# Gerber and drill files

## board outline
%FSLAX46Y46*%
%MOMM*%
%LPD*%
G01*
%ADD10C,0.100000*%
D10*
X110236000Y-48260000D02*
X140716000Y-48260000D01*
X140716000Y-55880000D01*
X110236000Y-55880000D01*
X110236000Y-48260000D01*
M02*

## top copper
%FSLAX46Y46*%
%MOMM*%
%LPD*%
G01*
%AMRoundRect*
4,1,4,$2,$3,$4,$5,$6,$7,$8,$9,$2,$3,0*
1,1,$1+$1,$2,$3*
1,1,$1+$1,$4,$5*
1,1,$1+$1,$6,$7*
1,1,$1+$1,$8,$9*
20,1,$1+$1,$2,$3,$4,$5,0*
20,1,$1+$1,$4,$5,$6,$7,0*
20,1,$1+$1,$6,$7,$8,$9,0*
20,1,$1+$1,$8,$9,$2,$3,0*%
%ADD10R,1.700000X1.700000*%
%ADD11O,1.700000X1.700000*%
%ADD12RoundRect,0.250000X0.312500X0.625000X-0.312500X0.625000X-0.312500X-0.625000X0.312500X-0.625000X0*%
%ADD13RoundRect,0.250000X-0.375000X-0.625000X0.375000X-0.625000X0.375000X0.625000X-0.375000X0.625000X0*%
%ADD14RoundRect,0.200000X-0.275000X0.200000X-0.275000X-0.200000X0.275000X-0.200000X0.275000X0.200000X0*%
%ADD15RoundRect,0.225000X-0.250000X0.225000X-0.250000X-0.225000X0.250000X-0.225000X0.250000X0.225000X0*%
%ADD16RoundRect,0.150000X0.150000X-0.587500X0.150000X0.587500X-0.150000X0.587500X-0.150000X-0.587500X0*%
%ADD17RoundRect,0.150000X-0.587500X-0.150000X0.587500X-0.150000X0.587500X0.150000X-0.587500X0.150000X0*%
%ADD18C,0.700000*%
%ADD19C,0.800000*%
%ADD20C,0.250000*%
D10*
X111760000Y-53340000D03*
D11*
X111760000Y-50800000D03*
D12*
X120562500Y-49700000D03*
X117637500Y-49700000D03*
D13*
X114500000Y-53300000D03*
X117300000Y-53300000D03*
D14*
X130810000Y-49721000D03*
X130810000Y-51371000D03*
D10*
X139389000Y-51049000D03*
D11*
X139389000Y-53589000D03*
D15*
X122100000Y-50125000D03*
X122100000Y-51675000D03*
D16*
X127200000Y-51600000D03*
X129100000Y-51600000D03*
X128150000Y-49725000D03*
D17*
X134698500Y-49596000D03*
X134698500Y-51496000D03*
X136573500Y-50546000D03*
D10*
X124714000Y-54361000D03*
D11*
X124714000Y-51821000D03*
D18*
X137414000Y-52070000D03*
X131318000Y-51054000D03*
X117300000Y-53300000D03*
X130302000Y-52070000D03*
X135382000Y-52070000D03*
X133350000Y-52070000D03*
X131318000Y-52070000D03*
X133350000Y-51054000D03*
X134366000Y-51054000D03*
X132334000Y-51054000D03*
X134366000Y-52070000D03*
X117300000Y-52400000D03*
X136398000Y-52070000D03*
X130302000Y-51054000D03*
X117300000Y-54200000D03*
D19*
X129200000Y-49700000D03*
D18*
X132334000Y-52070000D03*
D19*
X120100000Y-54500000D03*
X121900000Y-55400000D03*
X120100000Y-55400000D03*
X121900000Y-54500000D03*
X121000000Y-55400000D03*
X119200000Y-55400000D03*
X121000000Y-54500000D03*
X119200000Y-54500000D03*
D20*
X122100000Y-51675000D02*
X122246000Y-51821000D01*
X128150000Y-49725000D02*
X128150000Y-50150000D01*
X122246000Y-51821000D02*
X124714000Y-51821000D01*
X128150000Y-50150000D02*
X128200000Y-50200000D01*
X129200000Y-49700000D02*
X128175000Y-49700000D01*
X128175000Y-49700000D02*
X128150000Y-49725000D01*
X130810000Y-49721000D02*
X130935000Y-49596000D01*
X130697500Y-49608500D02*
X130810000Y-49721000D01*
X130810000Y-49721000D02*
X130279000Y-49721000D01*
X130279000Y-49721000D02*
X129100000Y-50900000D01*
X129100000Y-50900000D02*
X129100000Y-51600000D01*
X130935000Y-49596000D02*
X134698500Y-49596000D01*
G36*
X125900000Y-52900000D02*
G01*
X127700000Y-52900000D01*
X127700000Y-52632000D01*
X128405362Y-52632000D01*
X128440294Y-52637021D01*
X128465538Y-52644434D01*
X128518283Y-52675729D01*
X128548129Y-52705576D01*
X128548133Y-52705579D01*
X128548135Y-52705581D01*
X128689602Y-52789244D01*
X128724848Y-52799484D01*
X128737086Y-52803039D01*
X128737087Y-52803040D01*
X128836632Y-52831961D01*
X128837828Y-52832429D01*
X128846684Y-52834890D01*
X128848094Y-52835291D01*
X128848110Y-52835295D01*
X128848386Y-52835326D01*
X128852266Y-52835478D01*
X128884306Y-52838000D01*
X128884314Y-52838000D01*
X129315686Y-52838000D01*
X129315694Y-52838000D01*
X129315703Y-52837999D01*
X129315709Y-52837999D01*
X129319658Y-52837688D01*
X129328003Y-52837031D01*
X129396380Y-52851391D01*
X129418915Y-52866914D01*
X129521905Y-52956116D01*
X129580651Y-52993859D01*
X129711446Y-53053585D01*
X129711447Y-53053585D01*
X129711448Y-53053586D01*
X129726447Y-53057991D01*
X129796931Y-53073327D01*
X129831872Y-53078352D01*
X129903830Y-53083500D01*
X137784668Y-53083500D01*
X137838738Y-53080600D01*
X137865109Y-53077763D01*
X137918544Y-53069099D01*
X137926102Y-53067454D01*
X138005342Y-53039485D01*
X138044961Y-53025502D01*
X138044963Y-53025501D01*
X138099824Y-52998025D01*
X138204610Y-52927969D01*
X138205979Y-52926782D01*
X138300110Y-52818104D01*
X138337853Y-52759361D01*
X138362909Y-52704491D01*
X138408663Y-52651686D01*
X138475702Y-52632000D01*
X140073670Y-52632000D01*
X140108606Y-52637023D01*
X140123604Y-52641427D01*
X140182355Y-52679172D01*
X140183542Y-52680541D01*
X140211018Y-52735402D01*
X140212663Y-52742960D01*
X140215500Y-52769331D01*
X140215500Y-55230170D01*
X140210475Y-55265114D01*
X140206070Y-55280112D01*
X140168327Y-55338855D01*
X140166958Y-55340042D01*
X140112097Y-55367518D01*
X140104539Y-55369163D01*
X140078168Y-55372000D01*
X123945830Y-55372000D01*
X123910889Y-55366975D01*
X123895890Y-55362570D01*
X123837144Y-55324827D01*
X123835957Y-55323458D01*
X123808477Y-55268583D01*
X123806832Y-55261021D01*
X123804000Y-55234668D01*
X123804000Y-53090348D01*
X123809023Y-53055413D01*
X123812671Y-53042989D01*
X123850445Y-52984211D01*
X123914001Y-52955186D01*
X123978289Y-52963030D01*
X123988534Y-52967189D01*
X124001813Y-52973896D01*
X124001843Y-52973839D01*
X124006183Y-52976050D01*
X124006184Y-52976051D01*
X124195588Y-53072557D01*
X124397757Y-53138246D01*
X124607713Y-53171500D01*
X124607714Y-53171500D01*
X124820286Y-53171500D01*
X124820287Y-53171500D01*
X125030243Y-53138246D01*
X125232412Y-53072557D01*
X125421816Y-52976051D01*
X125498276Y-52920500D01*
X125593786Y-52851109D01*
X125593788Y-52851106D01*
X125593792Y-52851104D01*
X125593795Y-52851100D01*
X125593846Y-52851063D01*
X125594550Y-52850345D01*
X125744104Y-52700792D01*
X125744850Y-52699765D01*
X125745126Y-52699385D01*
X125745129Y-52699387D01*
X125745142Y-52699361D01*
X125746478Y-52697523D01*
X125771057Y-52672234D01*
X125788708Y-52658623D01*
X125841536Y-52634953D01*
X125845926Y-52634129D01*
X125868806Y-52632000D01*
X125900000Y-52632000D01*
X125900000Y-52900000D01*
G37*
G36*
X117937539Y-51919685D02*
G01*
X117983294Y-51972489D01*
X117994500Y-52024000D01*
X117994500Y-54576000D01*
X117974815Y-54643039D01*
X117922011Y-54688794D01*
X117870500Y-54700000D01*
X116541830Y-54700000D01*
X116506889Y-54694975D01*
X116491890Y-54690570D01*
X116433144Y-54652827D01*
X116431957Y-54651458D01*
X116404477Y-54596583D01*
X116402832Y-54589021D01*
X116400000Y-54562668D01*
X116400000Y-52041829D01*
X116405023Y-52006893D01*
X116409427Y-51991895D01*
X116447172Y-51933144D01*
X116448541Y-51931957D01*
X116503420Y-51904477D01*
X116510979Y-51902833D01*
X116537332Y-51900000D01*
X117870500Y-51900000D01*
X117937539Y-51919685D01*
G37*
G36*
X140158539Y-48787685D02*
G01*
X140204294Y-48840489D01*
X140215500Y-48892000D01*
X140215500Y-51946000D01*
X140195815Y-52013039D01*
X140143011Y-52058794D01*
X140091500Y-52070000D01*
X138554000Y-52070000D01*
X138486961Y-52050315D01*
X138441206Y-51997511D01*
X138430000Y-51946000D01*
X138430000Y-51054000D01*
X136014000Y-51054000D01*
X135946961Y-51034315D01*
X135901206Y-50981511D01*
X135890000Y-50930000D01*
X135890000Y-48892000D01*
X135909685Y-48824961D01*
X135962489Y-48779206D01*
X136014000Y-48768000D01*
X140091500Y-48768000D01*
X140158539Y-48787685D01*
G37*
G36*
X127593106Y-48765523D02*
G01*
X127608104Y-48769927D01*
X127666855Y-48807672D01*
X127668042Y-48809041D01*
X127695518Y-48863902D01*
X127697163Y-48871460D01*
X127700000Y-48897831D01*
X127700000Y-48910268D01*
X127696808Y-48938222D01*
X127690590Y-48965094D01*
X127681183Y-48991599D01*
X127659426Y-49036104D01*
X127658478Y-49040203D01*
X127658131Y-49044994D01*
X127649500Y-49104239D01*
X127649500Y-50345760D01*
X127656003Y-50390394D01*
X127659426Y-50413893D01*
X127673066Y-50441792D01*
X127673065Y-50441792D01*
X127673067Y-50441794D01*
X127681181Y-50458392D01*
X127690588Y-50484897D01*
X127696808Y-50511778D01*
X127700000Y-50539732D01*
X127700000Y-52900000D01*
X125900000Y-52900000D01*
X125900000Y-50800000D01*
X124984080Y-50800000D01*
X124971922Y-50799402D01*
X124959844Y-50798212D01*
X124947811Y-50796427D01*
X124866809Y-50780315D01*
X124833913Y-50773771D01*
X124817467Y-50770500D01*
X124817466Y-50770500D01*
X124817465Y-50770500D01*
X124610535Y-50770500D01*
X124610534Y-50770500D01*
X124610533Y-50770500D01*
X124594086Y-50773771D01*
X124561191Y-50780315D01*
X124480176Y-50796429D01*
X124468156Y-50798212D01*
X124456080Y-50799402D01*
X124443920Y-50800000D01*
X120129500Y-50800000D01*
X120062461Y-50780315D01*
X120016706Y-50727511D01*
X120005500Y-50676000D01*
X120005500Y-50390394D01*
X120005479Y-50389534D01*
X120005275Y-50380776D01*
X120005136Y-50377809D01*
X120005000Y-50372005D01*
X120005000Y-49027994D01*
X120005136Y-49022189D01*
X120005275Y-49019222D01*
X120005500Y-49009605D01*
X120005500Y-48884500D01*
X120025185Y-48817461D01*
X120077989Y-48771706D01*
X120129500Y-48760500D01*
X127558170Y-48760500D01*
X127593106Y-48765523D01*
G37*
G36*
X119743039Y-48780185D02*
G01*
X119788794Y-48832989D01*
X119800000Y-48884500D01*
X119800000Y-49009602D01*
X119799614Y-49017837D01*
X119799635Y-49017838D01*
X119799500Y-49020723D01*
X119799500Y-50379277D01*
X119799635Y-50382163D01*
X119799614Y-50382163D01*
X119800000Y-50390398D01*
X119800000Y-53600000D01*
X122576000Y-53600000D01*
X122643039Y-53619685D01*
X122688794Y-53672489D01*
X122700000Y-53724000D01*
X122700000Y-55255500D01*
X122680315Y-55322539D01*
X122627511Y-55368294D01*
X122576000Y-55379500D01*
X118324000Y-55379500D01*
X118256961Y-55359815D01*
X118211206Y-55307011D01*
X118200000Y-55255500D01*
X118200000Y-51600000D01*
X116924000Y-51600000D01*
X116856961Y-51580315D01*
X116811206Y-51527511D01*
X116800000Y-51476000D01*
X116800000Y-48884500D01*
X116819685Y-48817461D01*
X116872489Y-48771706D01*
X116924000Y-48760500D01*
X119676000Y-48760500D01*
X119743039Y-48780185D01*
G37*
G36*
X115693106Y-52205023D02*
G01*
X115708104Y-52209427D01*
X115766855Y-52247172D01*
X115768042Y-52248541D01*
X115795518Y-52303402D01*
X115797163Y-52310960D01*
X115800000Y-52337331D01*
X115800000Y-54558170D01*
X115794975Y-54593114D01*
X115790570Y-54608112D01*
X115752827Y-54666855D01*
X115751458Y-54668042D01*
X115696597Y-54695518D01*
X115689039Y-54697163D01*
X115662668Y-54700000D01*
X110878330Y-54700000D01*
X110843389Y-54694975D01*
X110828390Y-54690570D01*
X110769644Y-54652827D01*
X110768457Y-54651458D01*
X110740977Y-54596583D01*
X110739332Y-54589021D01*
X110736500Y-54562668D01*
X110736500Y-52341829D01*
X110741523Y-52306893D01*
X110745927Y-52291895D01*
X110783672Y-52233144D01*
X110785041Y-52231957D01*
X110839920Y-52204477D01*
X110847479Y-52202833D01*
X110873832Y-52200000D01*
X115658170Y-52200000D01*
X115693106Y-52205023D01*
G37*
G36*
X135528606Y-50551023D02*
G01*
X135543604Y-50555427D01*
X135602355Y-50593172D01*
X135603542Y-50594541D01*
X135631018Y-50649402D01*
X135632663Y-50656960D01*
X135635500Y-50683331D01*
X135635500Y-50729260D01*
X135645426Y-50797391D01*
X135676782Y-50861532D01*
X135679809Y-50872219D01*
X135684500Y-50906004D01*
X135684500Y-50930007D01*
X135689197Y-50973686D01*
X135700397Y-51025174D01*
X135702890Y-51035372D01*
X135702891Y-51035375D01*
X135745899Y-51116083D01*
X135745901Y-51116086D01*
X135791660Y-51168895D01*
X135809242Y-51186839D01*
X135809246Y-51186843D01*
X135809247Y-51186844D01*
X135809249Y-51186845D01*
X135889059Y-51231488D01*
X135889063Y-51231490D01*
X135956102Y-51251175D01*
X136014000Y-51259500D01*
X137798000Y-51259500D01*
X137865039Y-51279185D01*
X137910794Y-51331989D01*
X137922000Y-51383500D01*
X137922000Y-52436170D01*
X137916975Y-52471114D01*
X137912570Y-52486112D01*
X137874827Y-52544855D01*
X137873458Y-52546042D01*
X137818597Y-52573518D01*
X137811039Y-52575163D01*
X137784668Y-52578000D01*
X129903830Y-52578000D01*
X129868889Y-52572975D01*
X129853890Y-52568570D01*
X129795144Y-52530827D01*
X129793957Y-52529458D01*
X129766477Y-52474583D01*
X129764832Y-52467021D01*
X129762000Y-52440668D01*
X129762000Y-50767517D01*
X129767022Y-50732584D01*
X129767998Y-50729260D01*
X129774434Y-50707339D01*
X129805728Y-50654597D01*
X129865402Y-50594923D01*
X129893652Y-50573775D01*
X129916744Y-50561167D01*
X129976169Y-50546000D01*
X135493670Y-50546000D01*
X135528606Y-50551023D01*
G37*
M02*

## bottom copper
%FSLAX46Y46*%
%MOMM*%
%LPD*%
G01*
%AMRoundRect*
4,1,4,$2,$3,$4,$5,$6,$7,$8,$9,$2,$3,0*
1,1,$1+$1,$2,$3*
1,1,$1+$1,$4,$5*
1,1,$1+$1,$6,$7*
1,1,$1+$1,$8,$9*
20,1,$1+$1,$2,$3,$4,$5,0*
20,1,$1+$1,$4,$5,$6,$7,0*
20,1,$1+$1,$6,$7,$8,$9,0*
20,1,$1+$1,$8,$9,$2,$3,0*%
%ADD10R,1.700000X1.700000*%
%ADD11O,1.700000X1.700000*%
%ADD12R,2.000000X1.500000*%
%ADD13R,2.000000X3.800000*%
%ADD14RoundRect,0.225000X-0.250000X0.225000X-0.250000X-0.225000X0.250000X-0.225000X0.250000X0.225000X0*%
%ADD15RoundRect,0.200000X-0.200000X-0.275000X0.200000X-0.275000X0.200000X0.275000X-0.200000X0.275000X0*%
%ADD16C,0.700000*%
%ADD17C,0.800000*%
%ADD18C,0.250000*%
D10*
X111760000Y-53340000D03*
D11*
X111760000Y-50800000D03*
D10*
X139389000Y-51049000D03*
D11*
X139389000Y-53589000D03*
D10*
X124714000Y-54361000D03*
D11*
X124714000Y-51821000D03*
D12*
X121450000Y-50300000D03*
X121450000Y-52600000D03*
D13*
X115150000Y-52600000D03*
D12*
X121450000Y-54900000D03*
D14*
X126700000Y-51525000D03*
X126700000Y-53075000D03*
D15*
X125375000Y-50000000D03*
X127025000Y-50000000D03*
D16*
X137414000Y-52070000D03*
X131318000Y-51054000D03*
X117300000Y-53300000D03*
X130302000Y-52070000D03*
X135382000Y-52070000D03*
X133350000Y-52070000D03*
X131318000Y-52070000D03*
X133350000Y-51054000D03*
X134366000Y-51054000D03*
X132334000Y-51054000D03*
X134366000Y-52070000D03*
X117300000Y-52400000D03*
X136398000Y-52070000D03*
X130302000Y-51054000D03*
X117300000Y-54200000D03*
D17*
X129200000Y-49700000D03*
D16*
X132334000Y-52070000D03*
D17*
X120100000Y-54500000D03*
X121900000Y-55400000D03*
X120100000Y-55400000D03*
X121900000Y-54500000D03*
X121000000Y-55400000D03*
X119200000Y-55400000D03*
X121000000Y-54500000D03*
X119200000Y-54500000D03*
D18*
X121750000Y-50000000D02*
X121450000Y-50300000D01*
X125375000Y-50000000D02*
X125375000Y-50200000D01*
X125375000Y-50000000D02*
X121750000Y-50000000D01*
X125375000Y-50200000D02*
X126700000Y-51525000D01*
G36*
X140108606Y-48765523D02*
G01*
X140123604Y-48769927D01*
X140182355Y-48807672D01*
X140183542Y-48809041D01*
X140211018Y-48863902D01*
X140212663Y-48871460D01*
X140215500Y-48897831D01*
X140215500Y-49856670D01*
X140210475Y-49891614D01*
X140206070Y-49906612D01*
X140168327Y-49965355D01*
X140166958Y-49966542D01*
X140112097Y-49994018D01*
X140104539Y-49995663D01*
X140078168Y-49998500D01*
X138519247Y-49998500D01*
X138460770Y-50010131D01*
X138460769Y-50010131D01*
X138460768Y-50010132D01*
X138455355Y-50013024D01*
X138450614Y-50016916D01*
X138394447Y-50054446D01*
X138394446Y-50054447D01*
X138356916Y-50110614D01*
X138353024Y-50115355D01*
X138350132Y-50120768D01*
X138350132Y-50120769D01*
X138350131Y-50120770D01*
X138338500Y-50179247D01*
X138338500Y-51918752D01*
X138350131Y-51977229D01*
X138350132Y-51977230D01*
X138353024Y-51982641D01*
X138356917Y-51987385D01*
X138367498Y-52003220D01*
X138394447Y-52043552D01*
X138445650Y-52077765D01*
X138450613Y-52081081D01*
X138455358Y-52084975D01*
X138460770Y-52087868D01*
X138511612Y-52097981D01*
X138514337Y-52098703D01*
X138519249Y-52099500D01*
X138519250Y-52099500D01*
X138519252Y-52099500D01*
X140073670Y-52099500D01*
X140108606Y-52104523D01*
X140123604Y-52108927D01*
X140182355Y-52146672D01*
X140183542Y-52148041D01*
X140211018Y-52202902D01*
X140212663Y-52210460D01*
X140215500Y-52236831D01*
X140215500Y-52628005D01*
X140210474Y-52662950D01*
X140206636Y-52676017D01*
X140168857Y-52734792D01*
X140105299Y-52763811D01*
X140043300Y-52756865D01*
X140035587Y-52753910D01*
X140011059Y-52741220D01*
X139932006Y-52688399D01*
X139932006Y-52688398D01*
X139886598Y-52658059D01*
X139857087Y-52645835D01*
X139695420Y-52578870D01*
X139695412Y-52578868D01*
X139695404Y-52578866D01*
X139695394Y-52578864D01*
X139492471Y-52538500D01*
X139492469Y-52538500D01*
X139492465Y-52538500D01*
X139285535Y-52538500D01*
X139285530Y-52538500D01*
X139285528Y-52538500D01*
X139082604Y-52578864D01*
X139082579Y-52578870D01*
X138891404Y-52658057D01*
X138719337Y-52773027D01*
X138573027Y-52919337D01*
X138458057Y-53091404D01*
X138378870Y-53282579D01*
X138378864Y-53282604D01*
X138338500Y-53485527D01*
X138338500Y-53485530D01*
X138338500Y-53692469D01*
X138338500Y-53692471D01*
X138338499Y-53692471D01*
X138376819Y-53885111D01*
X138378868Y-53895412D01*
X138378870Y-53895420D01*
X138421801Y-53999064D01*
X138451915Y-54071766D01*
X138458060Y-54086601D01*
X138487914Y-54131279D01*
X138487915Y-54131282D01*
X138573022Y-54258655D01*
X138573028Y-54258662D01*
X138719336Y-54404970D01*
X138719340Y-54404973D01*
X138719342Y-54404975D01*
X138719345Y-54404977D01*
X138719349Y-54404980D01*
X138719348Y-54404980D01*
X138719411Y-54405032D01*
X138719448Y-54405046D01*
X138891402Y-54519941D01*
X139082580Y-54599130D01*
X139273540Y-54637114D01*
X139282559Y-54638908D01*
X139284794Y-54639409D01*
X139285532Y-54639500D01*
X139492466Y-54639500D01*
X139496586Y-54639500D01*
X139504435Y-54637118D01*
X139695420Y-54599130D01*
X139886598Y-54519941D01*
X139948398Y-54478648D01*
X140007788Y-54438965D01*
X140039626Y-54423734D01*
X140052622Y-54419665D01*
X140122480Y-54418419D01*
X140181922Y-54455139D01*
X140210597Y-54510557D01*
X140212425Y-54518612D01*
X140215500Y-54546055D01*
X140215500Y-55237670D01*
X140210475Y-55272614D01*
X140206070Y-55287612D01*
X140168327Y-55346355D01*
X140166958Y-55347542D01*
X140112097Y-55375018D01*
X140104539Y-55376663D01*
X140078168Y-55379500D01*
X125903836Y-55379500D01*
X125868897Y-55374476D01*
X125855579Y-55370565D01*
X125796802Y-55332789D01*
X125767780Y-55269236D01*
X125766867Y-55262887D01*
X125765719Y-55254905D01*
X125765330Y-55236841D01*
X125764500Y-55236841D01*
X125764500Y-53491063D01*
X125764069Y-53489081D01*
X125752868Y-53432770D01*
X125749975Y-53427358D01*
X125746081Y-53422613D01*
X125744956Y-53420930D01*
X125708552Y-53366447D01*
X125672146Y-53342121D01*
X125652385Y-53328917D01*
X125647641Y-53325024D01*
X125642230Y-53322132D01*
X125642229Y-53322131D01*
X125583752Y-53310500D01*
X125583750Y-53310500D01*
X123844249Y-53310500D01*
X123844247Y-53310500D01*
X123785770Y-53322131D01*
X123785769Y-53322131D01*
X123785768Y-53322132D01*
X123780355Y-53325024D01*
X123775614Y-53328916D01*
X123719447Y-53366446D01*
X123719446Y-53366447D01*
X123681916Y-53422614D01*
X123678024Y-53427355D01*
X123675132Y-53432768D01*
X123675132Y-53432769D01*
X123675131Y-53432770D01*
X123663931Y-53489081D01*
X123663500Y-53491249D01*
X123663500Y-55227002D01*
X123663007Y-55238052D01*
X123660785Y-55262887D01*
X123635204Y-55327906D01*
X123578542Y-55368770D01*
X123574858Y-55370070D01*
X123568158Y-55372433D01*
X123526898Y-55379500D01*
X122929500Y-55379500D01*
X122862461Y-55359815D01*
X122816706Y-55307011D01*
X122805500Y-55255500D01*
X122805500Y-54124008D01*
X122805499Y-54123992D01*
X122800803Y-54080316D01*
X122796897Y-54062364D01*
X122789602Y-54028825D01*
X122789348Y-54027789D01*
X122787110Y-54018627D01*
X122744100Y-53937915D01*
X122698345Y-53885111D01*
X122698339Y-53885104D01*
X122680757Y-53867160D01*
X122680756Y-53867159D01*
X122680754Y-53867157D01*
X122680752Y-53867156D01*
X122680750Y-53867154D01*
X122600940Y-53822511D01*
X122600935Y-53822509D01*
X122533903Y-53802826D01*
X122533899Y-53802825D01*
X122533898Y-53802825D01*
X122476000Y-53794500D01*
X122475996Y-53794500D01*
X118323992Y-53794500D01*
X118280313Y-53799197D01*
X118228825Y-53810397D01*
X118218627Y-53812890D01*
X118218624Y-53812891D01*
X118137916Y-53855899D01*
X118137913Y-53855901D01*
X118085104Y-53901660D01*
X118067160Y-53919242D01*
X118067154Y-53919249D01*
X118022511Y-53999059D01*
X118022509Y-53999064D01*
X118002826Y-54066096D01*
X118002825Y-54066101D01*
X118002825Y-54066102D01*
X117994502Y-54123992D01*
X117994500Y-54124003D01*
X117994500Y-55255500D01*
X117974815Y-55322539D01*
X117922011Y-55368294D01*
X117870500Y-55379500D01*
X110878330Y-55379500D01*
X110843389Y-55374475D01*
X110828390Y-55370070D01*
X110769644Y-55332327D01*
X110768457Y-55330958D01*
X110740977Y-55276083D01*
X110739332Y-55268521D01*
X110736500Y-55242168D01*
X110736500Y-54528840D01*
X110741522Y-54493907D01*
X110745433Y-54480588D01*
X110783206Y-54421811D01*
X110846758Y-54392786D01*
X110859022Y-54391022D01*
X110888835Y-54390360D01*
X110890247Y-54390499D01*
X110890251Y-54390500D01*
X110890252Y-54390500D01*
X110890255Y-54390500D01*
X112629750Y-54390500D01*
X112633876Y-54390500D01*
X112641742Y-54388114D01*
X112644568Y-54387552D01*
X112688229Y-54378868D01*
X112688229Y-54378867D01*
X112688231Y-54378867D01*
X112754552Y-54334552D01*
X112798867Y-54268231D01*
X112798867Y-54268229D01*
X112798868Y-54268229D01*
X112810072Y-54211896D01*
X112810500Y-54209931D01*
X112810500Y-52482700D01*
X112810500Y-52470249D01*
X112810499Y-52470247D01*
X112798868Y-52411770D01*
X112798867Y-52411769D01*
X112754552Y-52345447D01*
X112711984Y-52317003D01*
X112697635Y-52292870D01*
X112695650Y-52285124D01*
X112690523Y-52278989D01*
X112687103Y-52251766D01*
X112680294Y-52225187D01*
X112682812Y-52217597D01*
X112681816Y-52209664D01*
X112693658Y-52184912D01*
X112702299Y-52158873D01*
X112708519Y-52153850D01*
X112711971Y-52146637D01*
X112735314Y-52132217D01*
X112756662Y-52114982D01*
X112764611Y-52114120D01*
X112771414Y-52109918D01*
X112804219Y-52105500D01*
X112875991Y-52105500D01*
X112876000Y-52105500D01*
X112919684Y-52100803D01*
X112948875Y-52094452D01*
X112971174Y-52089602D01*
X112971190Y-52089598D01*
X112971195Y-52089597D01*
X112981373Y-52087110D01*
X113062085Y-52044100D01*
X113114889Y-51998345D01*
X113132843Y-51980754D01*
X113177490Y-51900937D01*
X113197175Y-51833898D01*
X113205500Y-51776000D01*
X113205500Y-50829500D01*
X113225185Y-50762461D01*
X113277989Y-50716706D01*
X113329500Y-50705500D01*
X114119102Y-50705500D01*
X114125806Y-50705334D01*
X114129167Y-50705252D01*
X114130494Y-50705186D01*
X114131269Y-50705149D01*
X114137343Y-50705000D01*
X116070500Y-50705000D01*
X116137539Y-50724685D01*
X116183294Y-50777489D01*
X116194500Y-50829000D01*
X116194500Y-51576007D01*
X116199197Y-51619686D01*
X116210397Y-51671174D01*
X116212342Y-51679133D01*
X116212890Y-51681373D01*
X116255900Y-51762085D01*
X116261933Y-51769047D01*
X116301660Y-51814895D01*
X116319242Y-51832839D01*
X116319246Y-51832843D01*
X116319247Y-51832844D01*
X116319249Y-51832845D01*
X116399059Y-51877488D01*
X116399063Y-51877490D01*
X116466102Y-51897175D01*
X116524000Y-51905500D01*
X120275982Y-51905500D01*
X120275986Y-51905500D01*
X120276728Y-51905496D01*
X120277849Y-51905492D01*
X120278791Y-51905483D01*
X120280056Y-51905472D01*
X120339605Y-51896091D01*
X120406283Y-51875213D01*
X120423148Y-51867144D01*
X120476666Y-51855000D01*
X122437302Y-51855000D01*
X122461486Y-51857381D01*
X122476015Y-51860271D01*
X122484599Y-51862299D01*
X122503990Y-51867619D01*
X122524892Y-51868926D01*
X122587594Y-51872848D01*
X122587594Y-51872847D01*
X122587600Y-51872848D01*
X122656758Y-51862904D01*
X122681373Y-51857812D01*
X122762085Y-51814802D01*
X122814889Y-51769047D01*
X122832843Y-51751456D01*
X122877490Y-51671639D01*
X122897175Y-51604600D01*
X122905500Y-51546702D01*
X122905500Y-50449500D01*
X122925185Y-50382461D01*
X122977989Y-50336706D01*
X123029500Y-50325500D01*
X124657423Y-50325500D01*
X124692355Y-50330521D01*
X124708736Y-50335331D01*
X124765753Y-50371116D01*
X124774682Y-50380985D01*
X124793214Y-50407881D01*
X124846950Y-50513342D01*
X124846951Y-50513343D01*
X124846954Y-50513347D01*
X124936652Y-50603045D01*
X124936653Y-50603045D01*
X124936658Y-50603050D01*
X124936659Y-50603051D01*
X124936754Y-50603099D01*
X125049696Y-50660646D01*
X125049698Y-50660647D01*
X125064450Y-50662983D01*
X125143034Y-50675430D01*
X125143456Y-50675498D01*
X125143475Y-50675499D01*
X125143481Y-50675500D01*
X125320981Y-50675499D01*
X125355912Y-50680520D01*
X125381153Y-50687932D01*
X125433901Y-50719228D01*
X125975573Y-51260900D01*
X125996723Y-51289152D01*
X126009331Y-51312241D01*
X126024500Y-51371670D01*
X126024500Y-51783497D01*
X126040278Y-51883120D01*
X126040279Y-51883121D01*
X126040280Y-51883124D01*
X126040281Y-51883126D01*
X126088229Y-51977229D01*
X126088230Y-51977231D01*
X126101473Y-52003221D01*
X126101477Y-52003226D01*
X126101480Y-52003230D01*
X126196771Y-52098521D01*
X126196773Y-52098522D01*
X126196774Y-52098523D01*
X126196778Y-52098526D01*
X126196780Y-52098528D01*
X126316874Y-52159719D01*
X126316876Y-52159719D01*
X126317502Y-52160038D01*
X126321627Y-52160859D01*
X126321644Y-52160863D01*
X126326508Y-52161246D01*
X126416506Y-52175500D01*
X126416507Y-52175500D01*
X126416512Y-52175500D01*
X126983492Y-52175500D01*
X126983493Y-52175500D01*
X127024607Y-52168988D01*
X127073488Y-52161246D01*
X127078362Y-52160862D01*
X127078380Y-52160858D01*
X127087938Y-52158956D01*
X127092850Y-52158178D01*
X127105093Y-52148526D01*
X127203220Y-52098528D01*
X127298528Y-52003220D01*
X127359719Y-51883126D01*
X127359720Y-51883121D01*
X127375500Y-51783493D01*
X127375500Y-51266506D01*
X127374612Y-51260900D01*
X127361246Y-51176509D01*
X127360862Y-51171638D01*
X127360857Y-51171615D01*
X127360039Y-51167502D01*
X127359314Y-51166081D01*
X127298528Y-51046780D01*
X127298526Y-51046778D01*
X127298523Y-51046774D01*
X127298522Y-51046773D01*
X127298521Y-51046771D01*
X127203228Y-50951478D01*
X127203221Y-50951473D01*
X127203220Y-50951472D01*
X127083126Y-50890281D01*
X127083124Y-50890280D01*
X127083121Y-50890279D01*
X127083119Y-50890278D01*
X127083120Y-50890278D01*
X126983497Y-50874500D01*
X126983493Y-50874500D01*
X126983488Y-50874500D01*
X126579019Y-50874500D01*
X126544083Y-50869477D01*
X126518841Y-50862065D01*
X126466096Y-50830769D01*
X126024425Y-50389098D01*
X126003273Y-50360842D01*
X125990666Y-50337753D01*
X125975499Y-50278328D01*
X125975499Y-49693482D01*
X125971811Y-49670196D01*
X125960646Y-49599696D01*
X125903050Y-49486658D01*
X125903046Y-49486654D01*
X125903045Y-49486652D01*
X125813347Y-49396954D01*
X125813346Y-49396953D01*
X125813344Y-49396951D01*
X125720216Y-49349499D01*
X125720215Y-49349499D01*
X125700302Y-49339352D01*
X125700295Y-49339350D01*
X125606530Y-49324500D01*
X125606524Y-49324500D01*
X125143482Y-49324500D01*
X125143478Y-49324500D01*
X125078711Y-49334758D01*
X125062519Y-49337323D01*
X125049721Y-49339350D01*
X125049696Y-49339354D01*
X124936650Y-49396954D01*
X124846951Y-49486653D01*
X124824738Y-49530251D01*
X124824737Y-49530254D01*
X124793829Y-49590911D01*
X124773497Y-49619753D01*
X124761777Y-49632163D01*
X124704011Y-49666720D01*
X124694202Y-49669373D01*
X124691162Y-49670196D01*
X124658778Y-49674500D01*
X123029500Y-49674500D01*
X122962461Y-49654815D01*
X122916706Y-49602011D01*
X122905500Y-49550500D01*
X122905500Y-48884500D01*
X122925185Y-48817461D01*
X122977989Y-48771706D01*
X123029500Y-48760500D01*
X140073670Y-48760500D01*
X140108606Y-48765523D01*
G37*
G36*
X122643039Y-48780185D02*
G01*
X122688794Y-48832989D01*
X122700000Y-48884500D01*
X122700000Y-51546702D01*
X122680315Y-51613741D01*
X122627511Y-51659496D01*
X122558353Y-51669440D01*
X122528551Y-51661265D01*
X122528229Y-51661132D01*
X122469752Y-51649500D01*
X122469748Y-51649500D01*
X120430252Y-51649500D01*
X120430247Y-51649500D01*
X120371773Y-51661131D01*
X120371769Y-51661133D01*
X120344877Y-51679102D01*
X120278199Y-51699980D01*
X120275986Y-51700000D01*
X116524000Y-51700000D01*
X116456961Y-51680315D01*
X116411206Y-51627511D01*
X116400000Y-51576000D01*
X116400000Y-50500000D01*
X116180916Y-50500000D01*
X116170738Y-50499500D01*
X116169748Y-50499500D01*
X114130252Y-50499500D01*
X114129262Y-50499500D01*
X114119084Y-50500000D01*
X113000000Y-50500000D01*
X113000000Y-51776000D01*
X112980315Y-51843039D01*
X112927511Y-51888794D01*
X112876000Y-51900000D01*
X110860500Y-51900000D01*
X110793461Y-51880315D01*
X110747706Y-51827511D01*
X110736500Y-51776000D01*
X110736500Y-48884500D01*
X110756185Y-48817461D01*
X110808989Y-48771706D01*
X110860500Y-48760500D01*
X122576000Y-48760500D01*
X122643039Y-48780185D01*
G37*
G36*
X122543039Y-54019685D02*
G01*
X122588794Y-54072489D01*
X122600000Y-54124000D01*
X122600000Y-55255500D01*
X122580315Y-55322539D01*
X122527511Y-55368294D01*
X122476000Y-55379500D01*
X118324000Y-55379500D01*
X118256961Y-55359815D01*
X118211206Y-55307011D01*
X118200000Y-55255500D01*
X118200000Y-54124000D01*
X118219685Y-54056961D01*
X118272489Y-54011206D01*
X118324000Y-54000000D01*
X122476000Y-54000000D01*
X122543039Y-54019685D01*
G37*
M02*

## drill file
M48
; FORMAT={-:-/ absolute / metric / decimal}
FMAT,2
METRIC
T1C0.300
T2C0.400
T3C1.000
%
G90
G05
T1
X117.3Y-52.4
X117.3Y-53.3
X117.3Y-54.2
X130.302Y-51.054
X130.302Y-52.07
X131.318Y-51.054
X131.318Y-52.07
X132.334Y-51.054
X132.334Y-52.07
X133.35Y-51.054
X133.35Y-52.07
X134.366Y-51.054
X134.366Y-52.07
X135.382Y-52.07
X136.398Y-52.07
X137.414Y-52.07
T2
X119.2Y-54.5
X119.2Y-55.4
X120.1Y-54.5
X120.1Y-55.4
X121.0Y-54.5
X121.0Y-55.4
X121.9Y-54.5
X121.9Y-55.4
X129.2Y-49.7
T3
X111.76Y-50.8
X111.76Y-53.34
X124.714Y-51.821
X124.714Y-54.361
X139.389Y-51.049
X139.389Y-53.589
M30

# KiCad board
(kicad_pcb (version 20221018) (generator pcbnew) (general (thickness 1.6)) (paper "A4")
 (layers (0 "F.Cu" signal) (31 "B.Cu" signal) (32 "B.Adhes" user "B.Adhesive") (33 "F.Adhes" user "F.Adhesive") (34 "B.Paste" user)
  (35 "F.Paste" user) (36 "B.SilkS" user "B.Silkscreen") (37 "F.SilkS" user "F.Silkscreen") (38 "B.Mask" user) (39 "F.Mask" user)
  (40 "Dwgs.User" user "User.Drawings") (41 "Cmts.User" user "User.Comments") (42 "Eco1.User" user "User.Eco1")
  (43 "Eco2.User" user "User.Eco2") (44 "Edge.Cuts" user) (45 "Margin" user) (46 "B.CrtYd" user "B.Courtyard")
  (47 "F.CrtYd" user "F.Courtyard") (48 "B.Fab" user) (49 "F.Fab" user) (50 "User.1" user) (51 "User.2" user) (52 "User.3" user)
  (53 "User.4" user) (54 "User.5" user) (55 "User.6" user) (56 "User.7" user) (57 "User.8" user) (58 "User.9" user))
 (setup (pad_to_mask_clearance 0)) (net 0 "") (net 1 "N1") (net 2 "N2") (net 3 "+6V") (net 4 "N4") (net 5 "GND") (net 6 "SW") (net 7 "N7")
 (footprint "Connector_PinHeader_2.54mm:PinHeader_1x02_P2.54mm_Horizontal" (layer "F.Cu") (at 111.76 53.34 180)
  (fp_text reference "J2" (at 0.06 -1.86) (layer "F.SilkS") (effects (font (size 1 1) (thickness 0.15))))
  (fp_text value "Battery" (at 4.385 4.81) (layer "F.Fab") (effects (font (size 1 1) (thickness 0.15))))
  (pad "1" thru_hole rect (at 0 0 180) (size 1.7 1.7) (drill 1) (layers "*.Cu" "*.Mask") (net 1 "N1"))
  (pad "2" thru_hole oval (at 0 2.54 180) (size 1.7 1.7) (drill 1) (layers "*.Cu" "*.Mask") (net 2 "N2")))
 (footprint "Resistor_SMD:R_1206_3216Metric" (layer "F.Cu") (at 119.1 49.7 180)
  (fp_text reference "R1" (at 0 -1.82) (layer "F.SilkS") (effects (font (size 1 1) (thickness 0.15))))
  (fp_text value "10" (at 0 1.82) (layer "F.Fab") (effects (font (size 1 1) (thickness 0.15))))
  (pad "1" smd roundrect (at -1.4625 0 180) (size 1.125 1.75) (layers "F.Cu" "F.Paste" "F.Mask") (roundrect_rratio 0.2222222222)
   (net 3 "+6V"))
  (pad "2" smd roundrect (at 1.4625 0 180) (size 1.125 1.75) (layers "F.Cu" "F.Paste" "F.Mask") (roundrect_rratio 0.2222222222) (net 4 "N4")))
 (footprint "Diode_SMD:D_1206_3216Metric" (layer "F.Cu") (at 115.9 53.3)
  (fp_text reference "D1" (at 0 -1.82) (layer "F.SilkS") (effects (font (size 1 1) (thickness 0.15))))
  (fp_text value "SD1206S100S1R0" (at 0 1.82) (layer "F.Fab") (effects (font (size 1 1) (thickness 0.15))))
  (pad "1" smd roundrect (at -1.4 0) (size 1.25 1.75) (layers "F.Cu" "F.Paste" "F.Mask") (roundrect_rratio 0.2) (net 1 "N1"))
  (pad "2" smd roundrect (at 1.4 0) (size 1.25 1.75) (layers "F.Cu" "F.Paste" "F.Mask") (roundrect_rratio 0.2) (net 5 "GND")))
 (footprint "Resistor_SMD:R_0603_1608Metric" (layer "F.Cu") (at 130.81 50.546 -90)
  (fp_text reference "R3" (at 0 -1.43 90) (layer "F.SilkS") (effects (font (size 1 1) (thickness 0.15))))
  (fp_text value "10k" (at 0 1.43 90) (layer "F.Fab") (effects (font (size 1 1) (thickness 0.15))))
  (pad "1" smd roundrect (at -0.825 0 270) (size 0.8 0.95) (layers "F.Cu" "F.Paste" "F.Mask") (roundrect_rratio 0.25) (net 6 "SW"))
  (pad "2" smd roundrect (at 0.825 0 270) (size 0.8 0.95) (layers "F.Cu" "F.Paste" "F.Mask") (roundrect_rratio 0.25) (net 5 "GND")))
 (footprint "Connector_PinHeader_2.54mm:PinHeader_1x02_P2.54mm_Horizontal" (layer "F.Cu") (at 139.389 51.049)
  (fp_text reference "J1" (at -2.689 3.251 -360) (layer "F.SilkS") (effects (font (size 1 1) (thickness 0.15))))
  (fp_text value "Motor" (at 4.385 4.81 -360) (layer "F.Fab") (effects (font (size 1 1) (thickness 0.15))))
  (pad "1" thru_hole rect (at 0 0) (size 1.7 1.7) (drill 1) (layers "*.Cu" "*.Mask") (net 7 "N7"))
  (pad "2" thru_hole oval (at 0 2.54) (size 1.7 1.7) (drill 1) (layers "*.Cu" "*.Mask") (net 3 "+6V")))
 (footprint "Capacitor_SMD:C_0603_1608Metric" (layer "F.Cu") (at 122.1 50.9 -90)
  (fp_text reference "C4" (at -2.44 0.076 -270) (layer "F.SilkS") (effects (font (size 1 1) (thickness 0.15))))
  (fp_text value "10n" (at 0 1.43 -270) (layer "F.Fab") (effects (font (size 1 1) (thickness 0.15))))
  (pad "1" smd roundrect (at -0.775 0 270) (size 0.9 0.95) (layers "F.Cu" "F.Paste" "F.Mask") (roundrect_rratio 0.25) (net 3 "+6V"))
  (pad "2" smd roundrect (at 0.775 0 270) (size 0.9 0.95) (layers "F.Cu" "F.Paste" "F.Mask") (roundrect_rratio 0.25) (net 5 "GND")))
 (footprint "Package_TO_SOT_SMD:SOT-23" (layer "F.Cu") (at 128.15 50.6625 90)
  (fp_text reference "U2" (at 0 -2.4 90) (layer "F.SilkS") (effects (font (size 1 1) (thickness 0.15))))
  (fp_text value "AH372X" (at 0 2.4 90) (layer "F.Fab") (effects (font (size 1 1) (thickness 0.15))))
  (pad "1" smd roundrect (at -0.9375 -0.95 90) (size 1.475 0.6) (layers "F.Cu" "F.Paste" "F.Mask") (roundrect_rratio 0.25) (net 3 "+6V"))
  (pad "2" smd roundrect (at -0.9375 0.95 90) (size 1.475 0.6) (layers "F.Cu" "F.Paste" "F.Mask") (roundrect_rratio 0.25) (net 6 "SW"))
  (pad "3" smd roundrect (at 0.9375 0 90) (size 1.475 0.6) (layers "F.Cu" "F.Paste" "F.Mask") (roundrect_rratio 0.25) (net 5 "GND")))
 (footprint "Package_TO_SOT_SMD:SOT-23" (layer "F.Cu") (at 135.636 50.546)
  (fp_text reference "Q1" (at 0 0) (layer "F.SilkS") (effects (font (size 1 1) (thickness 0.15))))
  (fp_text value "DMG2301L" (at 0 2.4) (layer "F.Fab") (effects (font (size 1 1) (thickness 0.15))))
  (pad "1" smd roundrect (at -0.9375 -0.95) (size 1.475 0.6) (layers "F.Cu" "F.Paste" "F.Mask") (roundrect_rratio 0.25) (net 6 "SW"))
  (pad "2" smd roundrect (at -0.9375 0.95) (size 1.475 0.6) (layers "F.Cu" "F.Paste" "F.Mask") (roundrect_rratio 0.25) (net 5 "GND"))
  (pad "3" smd roundrect (at 0.9375 0) (size 1.475 0.6) (layers "F.Cu" "F.Paste" "F.Mask") (roundrect_rratio 0.25) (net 7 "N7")))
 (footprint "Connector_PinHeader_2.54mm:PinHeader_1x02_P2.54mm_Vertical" (layer "F.Cu") (at 124.714 54.361 180)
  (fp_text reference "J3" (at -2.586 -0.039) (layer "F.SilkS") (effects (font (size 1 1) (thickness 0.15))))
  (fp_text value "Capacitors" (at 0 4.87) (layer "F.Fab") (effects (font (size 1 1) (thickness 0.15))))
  (pad "1" thru_hole rect (at 0 0 180) (size 1.7 1.7) (drill 1) (layers "*.Cu" "*.Mask") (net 3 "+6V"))
  (pad "2" thru_hole oval (at 0 2.54 180) (size 1.7 1.7) (drill 1) (layers "*.Cu" "*.Mask") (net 5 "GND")))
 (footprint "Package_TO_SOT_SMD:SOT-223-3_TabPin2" (layer "B.Cu") (at 118.3 52.6 180)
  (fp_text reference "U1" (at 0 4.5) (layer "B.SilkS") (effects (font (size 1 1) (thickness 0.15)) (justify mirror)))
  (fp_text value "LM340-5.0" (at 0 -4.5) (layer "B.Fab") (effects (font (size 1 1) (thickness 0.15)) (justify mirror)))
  (pad "1" smd rect (at -3.15 2.3 180) (size 2 1.5) (layers "B.Cu" "B.Paste" "B.Mask") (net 2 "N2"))
  (pad "2" smd rect (at -3.15 0 180) (size 2 1.5) (layers "B.Cu" "B.Paste" "B.Mask") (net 5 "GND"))
  (pad "2" smd rect (at 3.15 0 180) (size 2 3.8) (layers "B.Cu" "B.Paste" "B.Mask") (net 5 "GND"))
  (pad "3" smd rect (at -3.15 -2.3 180) (size 2 1.5) (layers "B.Cu" "B.Paste" "B.Mask") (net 4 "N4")))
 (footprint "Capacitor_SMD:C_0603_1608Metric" (layer "B.Cu") (at 126.7 52.3 -90)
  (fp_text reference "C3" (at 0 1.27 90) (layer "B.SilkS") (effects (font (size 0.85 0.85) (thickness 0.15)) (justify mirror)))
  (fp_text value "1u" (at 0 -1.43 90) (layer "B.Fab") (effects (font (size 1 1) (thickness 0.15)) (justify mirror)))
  (pad "1" smd roundrect (at -0.775 0 270) (size 0.9 0.95) (layers "B.Cu" "B.Paste" "B.Mask") (roundrect_rratio 0.25) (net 2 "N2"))
  (pad "2" smd roundrect (at 0.775 0 270) (size 0.9 0.95) (layers "B.Cu" "B.Paste" "B.Mask") (roundrect_rratio 0.25) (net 5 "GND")))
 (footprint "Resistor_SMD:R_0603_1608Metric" (layer "B.Cu") (at 126.2 50)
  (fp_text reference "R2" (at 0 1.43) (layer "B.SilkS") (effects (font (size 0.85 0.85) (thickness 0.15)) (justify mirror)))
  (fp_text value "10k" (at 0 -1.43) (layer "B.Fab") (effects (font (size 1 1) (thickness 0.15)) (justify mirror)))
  (pad "1" smd roundrect (at -0.825 0) (size 0.8 0.95) (layers "B.Cu" "B.Paste" "B.Mask") (roundrect_rratio 0.25) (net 2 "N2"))
  (pad "2" smd roundrect (at 0.825 0) (size 0.8 0.95) (layers "B.Cu" "B.Paste" "B.Mask") (roundrect_rratio 0.25) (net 5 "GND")))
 (gr_rect (start 110.236 48.26) (end 140.716 55.88) (stroke (width 0.1) (type default)) (fill none) (layer "Edge.Cuts"))
 (segment (start 122.1 51.675) (end 122.246 51.821) (width 0.25) (layer "F.Cu") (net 5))
 (segment (start 128.15 49.725) (end 128.15 50.15) (width 0.25) (layer "F.Cu") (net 5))
 (segment (start 122.246 51.821) (end 124.714 51.821) (width 0.25) (layer "F.Cu") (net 5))
 (segment (start 128.15 50.15) (end 128.2 50.2) (width 0.25) (layer "F.Cu") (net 5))
 (segment (start 129.2 49.7) (end 128.175 49.7) (width 0.25) (layer "F.Cu") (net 5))
 (segment (start 128.175 49.7) (end 128.15 49.725) (width 0.25) (layer "F.Cu") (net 5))
 (via (at 137.414 52.07) (size 0.7) (drill 0.3) (layers "F.Cu" "B.Cu") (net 5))
 (via (at 131.318 51.054) (size 0.7) (drill 0.3) (layers "F.Cu" "B.Cu") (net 5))
 (via (at 117.3 53.3) (size 0.7) (drill 0.3) (layers "F.Cu" "B.Cu") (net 5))
 (via (at 130.302 52.07) (size 0.7) (drill 0.3) (layers "F.Cu" "B.Cu") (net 5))
 (via (at 135.382 52.07) (size 0.7) (drill 0.3) (layers "F.Cu" "B.Cu") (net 5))
 (via (at 133.35 52.07) (size 0.7) (drill 0.3) (layers "F.Cu" "B.Cu") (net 5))
 (via (at 131.318 52.07) (size 0.7) (drill 0.3) (layers "F.Cu" "B.Cu") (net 5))
 (via (at 133.35 51.054) (size 0.7) (drill 0.3) (layers "F.Cu" "B.Cu") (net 5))
 (via (at 134.366 51.054) (size 0.7) (drill 0.3) (layers "F.Cu" "B.Cu") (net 5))
 (via (at 132.334 51.054) (size 0.7) (drill 0.3) (layers "F.Cu" "B.Cu") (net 5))
 (via (at 134.366 52.07) (size 0.7) (drill 0.3) (layers "F.Cu" "B.Cu") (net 5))
 (via (at 117.3 52.4) (size 0.7) (drill 0.3) (layers "F.Cu" "B.Cu") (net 5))
 (via (at 136.398 52.07) (size 0.7) (drill 0.3) (layers "F.Cu" "B.Cu") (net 5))
 (via (at 130.302 51.054) (size 0.7) (drill 0.3) (layers "F.Cu" "B.Cu") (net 5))
 (via (at 117.3 54.2) (size 0.7) (drill 0.3) (layers "F.Cu" "B.Cu") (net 5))
 (via (at 129.2 49.7) (size 0.8) (drill 0.4) (layers "F.Cu" "B.Cu") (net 5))
 (via (at 132.334 52.07) (size 0.7) (drill 0.3) (layers "F.Cu" "B.Cu") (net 5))
 (segment (start 130.81 49.721) (end 130.935 49.596) (width 0.25) (layer "F.Cu") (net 6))
 (segment (start 130.6975 49.6085) (end 130.81 49.721) (width 0.25) (layer "F.Cu") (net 6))
 (segment (start 130.81 49.721) (end 130.279 49.721) (width 0.25) (layer "F.Cu") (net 6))
 (segment (start 130.279 49.721) (end 129.1 50.9) (width 0.25) (layer "F.Cu") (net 6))
 (segment (start 129.1 50.9) (end 129.1 51.6) (width 0.25) (layer "F.Cu") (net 6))
 (segment (start 130.935 49.596) (end 134.6985 49.596) (width 0.25) (layer "F.Cu") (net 6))
 (segment (start 121.75 50) (end 121.45 50.3) (width 0.25) (layer "B.Cu") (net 2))
 (segment (start 125.375 50) (end 125.375 50.2) (width 0.25) (layer "B.Cu") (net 2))
 (segment (start 125.375 50) (end 121.75 50) (width 0.25) (layer "B.Cu") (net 2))
 (segment (start 125.375 50.2) (end 126.7 51.525) (width 0.25) (layer "B.Cu") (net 2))
 (via (at 120.1 54.5) (size 0.8) (drill 0.4) (layers "F.Cu" "B.Cu") (free) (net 4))
 (via (at 121.9 55.4) (size 0.8) (drill 0.4) (layers "F.Cu" "B.Cu") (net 4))
 (via (at 120.1 55.4) (size 0.8) (drill 0.4) (layers "F.Cu" "B.Cu") (free) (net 4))
 (via (at 121.9 54.5) (size 0.8) (drill 0.4) (layers "F.Cu" "B.Cu") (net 4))
 (via (at 121 55.4) (size 0.8) (drill 0.4) (layers "F.Cu" "B.Cu") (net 4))
 (via (at 119.2 55.4) (size 0.8) (drill 0.4) (layers "F.Cu" "B.Cu") (free) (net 4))
 (via (at 121 54.5) (size 0.8) (drill 0.4) (layers "F.Cu" "B.Cu") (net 4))
 (via (at 119.2 54.5) (size 0.8) (drill 0.4) (layers "F.Cu" "B.Cu") (free) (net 4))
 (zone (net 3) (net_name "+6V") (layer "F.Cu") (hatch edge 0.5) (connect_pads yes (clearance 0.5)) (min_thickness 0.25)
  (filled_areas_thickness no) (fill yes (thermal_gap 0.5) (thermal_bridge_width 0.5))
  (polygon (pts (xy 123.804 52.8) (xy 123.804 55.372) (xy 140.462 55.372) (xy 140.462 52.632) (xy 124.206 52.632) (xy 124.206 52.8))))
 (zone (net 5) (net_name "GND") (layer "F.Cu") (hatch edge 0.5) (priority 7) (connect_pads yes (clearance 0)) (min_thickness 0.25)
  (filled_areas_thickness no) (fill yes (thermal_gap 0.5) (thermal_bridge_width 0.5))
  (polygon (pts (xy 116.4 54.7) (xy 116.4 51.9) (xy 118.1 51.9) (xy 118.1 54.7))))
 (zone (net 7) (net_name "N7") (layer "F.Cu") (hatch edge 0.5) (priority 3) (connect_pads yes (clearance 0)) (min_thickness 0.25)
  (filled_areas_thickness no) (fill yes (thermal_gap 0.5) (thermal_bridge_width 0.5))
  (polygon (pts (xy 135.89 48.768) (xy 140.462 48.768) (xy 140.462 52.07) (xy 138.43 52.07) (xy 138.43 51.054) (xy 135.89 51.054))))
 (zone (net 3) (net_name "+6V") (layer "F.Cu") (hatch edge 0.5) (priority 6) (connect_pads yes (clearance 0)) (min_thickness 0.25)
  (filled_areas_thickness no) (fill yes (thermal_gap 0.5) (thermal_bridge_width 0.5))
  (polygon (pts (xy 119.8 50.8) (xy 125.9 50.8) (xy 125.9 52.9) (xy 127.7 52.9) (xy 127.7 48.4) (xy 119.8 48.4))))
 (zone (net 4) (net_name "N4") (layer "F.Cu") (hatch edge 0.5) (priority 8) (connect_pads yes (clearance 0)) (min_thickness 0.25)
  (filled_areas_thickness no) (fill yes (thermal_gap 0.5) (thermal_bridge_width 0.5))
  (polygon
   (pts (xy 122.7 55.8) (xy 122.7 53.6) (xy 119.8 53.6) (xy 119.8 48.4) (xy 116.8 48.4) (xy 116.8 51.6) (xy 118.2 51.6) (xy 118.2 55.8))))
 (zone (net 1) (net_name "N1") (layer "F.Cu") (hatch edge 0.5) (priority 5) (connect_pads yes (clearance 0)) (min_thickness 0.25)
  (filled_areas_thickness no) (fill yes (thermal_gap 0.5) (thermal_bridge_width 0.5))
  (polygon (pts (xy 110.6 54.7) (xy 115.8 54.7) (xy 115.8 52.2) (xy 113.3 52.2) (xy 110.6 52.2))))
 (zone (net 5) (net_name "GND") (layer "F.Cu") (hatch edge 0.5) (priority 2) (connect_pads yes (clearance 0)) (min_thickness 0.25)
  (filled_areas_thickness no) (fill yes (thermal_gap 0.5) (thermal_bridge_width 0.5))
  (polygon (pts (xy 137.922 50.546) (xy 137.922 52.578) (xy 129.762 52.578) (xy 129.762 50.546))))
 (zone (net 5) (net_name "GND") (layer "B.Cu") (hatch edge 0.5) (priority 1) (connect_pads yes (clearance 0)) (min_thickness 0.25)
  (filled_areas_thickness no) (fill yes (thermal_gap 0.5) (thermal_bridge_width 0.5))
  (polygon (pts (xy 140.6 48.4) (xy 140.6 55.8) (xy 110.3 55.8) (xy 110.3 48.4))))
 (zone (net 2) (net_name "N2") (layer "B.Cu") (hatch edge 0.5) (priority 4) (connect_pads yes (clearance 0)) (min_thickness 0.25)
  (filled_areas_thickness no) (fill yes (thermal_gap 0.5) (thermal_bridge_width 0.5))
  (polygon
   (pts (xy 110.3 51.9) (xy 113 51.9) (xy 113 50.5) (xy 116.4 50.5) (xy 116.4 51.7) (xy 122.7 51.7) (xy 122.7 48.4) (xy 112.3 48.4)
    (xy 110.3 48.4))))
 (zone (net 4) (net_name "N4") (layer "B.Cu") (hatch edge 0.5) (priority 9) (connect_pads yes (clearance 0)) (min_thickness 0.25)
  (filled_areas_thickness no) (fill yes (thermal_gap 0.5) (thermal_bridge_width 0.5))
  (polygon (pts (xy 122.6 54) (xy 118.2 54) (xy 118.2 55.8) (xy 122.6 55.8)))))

